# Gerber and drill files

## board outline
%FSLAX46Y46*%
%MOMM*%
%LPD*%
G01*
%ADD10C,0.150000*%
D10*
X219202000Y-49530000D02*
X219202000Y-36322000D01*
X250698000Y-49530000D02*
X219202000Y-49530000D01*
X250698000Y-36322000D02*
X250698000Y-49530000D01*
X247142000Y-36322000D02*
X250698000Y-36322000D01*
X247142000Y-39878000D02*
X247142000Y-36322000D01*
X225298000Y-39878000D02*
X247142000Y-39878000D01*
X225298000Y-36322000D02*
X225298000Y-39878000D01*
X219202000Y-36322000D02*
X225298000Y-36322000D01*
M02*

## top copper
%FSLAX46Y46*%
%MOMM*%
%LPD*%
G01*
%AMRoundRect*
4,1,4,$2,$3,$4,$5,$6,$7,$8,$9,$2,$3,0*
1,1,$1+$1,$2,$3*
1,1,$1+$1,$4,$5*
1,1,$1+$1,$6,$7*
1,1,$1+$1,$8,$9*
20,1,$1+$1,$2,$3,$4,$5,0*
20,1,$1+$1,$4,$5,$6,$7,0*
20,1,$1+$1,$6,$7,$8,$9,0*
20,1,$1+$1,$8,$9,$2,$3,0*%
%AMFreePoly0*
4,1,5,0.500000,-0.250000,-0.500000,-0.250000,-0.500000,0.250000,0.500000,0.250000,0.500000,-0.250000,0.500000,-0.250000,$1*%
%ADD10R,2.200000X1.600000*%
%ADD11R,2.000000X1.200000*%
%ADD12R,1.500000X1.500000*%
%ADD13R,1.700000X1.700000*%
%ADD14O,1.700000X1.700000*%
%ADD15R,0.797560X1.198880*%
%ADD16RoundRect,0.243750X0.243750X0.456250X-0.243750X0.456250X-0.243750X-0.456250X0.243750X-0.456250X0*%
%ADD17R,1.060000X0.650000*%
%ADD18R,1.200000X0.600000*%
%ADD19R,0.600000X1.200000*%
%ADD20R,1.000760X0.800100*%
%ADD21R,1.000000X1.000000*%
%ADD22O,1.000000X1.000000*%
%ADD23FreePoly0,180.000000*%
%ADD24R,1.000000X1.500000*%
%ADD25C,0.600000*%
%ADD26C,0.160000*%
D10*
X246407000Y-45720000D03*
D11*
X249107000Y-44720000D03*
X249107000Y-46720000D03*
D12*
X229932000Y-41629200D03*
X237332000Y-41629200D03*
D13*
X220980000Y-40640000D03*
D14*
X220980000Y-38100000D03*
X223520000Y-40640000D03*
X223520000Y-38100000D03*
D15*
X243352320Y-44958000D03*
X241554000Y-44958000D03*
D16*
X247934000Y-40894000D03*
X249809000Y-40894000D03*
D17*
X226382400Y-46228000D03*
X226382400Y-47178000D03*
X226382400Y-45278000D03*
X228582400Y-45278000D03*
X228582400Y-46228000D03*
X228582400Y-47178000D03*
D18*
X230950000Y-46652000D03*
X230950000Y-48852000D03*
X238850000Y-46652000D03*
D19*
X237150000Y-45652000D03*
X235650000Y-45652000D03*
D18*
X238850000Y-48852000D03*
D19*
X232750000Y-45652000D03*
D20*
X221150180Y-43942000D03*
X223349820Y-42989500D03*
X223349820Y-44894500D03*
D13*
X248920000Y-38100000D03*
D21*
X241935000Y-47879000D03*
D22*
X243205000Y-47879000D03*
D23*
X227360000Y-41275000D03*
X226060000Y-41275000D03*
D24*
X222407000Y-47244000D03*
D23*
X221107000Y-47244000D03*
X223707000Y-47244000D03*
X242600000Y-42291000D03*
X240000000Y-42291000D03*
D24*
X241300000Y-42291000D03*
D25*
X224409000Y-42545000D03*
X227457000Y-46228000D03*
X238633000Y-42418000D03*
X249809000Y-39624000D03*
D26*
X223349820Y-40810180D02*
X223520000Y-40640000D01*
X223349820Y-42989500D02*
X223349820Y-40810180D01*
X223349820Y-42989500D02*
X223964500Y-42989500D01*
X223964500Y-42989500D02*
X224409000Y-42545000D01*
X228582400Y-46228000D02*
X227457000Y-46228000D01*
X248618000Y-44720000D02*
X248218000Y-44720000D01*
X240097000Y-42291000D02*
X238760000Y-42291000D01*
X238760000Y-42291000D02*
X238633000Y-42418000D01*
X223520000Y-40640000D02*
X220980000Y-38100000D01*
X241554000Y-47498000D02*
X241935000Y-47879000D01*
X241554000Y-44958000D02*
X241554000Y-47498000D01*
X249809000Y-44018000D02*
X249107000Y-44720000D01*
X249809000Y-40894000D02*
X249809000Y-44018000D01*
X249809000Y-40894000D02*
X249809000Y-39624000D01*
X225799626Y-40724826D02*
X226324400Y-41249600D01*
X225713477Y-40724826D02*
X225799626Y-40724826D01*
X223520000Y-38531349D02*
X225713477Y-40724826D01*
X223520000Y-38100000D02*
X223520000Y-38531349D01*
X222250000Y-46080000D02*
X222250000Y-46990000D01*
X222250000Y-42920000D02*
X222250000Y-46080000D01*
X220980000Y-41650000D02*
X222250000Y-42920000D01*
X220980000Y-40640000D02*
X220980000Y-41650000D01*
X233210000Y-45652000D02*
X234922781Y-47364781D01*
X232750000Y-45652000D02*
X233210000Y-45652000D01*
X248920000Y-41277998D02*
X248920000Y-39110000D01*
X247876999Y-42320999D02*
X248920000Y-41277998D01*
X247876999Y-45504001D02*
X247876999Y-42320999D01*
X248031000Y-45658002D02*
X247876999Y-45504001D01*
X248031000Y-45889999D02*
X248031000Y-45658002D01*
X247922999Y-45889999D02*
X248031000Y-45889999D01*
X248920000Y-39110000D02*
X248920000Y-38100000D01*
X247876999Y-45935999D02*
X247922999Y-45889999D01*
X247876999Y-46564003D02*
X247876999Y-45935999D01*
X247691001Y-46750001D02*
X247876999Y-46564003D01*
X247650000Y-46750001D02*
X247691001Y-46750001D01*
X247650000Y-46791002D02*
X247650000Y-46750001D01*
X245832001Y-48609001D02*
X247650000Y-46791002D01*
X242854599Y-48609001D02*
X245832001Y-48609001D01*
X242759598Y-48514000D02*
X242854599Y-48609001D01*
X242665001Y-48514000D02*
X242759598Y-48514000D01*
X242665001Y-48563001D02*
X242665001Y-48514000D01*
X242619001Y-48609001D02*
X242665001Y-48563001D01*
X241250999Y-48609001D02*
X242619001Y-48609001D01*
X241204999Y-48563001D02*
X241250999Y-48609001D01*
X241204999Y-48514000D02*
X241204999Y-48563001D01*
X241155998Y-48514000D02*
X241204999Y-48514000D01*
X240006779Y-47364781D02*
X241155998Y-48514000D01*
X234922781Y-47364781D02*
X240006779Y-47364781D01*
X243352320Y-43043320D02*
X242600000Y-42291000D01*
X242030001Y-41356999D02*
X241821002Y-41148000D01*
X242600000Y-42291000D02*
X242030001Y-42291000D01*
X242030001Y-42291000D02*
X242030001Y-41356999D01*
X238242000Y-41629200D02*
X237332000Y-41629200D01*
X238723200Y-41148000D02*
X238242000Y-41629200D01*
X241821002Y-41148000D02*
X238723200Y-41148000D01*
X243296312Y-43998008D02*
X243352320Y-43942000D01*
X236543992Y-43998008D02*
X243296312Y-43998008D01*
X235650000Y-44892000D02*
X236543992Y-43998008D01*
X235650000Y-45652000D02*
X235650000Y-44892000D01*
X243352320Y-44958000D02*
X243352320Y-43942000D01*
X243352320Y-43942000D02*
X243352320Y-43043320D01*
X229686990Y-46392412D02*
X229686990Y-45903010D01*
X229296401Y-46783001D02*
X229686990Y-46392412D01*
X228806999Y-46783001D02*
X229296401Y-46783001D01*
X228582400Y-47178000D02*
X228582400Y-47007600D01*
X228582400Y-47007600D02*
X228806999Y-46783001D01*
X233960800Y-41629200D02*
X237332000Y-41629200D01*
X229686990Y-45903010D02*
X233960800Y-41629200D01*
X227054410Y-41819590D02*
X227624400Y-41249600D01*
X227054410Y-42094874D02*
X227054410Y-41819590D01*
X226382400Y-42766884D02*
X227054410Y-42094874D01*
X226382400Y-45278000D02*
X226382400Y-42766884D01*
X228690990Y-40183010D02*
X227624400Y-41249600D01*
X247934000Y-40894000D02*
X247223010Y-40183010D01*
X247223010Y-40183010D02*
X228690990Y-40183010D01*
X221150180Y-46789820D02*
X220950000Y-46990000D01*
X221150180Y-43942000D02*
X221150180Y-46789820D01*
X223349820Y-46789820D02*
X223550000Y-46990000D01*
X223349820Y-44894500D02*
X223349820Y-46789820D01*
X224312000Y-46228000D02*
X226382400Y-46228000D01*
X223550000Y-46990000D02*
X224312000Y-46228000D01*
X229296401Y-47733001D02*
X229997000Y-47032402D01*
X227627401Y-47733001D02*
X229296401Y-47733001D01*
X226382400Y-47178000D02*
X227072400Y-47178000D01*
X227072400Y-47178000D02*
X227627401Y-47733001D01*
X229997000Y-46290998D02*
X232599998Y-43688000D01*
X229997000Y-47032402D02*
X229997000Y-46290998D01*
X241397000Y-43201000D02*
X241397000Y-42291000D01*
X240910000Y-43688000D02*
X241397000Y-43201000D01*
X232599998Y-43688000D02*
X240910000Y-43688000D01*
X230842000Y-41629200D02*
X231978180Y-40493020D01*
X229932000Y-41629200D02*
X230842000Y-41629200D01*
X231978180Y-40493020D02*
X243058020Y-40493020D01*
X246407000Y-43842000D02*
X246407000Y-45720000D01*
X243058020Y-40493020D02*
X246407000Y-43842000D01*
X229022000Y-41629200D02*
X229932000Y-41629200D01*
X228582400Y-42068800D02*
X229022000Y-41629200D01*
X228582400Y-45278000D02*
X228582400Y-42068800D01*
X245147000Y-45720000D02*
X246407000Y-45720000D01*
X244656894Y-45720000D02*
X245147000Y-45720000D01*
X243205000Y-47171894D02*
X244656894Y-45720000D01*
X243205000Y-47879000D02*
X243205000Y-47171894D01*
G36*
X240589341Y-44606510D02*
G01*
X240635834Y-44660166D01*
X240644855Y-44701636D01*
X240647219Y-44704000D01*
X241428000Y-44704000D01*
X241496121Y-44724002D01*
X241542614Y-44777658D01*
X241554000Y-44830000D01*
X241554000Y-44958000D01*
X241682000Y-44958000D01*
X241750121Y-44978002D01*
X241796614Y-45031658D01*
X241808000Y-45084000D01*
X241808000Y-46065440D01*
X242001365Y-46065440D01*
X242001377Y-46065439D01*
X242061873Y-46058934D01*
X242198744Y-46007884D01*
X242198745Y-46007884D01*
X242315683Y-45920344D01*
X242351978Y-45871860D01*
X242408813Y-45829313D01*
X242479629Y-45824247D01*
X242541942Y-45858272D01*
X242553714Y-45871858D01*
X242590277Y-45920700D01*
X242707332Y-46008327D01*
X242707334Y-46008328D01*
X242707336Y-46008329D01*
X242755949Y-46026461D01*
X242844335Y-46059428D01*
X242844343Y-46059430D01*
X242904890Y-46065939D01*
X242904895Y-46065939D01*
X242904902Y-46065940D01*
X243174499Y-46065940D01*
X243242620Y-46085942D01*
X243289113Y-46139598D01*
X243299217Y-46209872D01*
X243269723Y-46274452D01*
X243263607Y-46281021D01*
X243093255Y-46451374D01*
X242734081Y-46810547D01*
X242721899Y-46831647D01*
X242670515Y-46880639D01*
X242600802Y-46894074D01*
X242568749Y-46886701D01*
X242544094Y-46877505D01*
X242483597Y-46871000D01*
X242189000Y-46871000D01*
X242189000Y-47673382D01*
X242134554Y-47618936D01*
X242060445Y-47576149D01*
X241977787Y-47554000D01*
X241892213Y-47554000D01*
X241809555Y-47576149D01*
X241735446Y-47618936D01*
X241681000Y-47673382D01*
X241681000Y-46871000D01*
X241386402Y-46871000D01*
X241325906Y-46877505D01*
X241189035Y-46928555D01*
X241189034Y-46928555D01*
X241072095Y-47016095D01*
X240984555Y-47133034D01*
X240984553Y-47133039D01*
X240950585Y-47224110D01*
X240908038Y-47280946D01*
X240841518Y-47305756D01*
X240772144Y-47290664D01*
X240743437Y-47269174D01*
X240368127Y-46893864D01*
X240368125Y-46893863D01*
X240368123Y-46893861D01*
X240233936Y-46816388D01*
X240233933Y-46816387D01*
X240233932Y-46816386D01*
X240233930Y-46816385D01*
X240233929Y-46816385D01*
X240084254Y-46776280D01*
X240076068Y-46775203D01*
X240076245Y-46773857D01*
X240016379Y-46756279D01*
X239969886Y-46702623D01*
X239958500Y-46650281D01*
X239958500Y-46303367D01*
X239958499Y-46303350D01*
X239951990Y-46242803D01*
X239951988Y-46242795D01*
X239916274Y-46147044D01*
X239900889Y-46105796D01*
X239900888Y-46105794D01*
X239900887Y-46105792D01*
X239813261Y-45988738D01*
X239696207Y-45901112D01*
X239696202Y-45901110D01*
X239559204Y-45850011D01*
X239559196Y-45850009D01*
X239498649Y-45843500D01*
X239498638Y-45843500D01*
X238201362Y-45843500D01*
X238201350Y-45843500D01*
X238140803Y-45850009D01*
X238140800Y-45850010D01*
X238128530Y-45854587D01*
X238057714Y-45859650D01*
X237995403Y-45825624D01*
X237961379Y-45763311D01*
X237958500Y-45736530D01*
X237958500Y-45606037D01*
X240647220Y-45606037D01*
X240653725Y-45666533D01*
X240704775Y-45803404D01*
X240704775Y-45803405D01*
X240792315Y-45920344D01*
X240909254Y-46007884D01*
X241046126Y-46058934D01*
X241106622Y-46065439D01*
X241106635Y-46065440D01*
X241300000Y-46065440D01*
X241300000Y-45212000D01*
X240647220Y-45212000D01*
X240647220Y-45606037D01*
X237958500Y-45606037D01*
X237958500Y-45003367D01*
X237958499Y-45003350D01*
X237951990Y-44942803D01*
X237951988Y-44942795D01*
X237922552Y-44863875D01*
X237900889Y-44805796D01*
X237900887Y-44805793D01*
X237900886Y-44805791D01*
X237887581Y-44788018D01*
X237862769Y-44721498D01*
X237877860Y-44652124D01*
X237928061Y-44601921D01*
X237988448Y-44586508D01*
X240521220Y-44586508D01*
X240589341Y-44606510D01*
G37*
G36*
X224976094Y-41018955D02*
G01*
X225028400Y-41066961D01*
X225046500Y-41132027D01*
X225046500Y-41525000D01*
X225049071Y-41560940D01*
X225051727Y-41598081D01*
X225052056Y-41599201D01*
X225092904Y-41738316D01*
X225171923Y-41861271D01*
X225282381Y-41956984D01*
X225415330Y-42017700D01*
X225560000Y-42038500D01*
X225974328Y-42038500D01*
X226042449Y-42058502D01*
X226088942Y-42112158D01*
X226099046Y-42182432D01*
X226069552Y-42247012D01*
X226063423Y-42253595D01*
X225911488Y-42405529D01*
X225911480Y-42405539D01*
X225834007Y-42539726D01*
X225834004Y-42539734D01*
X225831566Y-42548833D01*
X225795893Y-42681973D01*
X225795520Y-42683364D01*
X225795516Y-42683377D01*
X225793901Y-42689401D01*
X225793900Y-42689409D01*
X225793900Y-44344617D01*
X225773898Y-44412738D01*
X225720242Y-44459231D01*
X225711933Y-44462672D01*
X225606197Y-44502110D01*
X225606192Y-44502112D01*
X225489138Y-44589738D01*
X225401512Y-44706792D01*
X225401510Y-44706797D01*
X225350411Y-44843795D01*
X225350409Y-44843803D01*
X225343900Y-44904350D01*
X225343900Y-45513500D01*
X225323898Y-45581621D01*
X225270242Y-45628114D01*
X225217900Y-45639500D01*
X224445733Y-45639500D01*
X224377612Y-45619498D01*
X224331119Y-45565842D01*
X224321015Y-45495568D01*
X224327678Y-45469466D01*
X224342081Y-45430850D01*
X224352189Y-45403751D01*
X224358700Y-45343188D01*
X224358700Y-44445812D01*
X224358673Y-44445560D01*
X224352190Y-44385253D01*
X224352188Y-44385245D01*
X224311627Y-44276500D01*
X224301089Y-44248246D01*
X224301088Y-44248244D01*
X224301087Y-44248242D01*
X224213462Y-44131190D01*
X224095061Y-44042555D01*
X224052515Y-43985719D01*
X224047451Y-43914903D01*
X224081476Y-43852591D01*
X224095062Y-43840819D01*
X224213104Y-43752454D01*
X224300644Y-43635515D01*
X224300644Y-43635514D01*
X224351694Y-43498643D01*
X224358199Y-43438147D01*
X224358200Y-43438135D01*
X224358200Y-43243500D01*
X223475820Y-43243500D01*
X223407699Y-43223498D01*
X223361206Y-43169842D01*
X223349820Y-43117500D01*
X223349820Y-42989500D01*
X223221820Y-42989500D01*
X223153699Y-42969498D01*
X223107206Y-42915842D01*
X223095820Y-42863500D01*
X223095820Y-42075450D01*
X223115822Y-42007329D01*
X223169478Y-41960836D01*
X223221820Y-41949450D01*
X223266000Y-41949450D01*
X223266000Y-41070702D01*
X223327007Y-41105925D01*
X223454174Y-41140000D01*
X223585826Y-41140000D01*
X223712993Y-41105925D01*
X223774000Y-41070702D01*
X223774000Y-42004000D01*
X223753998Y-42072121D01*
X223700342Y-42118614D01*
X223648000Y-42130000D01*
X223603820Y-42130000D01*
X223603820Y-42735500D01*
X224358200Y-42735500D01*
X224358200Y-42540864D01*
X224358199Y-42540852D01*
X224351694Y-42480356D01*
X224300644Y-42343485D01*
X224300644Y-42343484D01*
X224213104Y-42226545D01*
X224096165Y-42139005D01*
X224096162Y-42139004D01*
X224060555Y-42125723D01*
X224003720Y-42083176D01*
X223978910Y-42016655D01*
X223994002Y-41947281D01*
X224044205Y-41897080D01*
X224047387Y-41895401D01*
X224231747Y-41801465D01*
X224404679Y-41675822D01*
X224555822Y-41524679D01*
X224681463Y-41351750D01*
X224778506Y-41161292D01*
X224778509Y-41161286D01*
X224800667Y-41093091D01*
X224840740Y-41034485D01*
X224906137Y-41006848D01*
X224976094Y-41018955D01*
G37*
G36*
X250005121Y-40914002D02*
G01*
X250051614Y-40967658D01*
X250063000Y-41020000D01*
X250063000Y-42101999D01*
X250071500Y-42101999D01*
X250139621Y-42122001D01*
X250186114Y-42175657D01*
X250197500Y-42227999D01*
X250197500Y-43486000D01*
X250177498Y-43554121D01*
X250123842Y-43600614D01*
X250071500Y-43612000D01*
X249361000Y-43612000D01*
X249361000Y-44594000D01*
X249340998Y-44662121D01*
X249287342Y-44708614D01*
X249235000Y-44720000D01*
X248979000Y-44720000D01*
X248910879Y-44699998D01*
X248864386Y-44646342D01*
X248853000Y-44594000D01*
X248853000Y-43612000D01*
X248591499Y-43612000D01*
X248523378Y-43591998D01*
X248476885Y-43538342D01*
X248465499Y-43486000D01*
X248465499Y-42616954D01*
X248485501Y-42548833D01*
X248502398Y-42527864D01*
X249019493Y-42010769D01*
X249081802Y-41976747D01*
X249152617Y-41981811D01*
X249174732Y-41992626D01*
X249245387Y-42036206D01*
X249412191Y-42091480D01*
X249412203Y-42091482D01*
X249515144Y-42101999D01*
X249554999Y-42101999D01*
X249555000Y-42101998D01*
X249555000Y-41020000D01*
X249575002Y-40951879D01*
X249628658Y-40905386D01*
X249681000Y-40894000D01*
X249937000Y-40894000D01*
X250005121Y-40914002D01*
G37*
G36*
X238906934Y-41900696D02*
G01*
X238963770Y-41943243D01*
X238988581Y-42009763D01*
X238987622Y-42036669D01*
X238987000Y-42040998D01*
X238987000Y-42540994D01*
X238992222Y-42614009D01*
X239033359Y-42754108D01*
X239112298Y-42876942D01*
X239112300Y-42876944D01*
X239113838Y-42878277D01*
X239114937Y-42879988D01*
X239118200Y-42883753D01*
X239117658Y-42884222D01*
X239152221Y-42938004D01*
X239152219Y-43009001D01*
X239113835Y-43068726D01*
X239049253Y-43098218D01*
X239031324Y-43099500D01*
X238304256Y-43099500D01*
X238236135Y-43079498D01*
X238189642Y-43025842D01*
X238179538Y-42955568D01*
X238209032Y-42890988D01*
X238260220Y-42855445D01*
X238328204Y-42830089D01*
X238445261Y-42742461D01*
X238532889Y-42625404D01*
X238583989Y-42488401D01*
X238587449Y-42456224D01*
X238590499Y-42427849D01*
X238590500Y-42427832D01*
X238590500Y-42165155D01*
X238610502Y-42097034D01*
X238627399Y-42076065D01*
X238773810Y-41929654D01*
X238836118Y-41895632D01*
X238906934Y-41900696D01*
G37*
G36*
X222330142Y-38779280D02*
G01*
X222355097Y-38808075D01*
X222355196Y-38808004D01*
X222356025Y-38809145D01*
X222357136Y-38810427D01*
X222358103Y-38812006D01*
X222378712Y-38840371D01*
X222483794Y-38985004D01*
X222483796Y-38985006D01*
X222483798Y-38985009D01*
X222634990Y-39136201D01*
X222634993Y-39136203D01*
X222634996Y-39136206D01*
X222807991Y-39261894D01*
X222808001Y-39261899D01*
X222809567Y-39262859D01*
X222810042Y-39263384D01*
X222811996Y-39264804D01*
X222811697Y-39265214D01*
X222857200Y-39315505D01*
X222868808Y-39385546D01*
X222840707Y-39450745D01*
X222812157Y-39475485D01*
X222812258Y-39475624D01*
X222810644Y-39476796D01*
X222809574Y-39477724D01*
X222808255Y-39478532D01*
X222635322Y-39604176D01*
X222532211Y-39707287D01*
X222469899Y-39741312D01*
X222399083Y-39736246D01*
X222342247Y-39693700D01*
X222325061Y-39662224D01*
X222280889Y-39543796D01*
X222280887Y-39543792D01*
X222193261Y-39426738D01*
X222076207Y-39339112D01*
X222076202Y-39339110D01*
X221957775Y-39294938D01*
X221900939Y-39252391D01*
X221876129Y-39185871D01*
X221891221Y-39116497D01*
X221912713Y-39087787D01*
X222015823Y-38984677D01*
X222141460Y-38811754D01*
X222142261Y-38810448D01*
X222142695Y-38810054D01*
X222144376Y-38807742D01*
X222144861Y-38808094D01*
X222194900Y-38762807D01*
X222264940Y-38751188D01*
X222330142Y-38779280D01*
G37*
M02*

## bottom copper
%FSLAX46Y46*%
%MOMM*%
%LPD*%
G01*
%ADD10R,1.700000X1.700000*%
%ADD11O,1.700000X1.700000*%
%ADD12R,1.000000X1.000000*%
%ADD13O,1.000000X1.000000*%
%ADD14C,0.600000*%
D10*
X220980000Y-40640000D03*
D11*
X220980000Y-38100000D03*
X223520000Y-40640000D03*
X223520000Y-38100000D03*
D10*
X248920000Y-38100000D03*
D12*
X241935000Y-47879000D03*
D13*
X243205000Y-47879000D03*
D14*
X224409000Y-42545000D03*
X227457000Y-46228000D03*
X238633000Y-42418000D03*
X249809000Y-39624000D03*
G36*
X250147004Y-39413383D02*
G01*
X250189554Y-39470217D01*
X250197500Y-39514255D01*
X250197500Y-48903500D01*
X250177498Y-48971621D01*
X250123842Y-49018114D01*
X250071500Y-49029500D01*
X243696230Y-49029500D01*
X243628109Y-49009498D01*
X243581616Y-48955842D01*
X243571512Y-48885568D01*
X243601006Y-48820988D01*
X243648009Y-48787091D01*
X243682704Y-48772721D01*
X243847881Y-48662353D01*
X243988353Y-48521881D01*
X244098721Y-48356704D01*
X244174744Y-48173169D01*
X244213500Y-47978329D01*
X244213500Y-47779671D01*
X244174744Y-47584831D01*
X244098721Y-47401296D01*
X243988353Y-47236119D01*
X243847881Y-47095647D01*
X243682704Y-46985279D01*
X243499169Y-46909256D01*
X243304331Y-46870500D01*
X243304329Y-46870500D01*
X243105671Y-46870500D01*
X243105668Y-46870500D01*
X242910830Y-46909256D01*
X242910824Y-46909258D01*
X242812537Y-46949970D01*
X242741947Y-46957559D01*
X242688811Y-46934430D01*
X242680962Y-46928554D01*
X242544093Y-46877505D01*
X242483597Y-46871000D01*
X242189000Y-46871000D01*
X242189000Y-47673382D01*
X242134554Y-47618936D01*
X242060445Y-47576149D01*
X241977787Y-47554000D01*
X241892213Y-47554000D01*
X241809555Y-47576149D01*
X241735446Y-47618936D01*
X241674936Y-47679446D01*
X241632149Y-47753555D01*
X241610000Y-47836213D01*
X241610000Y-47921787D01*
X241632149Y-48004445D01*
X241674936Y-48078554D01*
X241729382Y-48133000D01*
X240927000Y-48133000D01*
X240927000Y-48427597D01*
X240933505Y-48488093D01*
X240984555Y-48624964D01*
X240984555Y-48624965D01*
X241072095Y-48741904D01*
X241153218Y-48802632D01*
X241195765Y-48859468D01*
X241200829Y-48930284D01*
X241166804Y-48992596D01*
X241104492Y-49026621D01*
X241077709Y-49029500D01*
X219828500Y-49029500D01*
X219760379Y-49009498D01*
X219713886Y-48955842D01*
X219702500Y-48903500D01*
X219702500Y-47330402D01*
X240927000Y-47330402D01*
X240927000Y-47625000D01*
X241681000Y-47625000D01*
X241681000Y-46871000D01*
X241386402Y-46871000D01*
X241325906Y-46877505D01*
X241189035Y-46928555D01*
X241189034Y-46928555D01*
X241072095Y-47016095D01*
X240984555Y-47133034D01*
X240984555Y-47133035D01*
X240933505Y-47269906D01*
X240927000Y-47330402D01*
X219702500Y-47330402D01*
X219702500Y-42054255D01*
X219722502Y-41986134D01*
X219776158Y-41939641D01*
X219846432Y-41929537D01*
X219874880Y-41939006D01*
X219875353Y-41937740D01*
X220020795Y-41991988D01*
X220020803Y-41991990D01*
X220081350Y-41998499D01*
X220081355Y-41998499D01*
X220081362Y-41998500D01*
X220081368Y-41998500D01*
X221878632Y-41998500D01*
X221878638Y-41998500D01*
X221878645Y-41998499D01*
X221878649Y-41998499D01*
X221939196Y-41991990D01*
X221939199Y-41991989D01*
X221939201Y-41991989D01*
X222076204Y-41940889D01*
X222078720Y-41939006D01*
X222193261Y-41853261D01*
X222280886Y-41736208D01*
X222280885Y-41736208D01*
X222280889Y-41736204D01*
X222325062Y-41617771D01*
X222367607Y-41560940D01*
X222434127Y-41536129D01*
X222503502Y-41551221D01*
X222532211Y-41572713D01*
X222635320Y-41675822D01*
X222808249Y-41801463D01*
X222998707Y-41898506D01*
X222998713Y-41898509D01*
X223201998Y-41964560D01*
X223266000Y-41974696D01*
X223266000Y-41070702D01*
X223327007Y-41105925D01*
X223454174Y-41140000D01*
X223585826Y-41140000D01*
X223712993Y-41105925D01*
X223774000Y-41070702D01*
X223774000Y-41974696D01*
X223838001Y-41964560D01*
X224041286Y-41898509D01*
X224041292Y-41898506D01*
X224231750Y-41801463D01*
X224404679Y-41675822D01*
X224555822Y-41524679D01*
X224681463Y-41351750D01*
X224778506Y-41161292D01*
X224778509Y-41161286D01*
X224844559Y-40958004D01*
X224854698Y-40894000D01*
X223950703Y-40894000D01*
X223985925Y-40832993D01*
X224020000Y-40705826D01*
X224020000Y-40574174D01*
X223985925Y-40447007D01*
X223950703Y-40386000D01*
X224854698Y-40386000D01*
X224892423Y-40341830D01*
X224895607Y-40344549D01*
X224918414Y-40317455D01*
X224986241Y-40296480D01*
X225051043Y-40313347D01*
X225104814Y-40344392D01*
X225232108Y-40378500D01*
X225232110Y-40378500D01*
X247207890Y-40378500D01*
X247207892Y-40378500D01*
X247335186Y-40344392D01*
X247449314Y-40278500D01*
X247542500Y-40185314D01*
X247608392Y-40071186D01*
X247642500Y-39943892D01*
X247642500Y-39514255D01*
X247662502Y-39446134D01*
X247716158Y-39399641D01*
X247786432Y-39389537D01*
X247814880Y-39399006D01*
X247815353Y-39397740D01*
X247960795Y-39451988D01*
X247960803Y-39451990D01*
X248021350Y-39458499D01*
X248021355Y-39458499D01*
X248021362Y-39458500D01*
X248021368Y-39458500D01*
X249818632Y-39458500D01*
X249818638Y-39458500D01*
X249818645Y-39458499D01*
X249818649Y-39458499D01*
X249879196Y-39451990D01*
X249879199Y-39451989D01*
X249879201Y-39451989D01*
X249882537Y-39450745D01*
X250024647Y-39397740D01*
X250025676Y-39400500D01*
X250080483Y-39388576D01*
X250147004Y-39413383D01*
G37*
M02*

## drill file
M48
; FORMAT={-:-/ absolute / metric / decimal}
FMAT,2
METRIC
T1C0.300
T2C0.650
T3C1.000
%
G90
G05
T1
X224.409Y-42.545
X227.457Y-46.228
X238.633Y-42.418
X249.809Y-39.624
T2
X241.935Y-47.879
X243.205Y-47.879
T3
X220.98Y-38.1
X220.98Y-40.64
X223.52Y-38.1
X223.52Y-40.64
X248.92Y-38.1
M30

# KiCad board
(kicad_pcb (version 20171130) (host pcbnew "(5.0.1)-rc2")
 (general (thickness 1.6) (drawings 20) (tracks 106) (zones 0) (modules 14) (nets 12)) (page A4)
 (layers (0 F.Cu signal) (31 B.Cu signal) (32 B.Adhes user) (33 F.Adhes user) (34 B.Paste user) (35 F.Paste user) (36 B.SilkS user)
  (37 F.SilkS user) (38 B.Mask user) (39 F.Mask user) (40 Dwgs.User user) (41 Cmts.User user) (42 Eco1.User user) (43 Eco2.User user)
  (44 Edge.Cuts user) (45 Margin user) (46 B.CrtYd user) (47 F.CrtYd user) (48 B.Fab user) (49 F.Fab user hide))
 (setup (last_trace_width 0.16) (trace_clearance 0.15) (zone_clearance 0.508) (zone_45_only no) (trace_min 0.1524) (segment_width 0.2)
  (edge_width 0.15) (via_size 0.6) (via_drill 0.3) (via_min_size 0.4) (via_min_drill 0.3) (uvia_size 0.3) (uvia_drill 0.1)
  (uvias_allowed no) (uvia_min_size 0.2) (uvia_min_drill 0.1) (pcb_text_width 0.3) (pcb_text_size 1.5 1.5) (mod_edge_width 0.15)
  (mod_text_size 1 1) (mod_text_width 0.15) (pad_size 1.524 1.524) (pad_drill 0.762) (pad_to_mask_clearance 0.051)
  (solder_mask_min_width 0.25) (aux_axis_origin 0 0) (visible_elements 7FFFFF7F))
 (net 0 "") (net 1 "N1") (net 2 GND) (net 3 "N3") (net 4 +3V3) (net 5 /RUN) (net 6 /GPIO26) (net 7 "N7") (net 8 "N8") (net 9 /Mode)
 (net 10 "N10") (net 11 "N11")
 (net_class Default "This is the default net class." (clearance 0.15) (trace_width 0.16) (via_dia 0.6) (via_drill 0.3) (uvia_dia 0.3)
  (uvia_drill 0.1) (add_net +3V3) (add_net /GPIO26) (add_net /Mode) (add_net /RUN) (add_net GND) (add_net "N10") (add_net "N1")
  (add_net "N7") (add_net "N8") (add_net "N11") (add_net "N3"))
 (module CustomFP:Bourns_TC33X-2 (layer F.Cu) (at 246.507 45.72 90)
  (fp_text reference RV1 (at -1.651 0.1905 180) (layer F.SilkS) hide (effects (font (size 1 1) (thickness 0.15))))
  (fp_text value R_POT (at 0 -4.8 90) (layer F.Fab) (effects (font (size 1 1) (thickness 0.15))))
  (pad 1 smd rect (at 0 -0.1 90) (size 1.6 2.2) (layers F.Cu F.Paste F.Mask) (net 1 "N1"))
  (pad 2 smd rect (at 1 2.6 90) (size 1.2 2) (layers F.Cu F.Paste F.Mask) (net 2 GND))
  (pad 3 smd rect (at -1 2.6 90) (size 1.2 2) (layers F.Cu F.Paste F.Mask) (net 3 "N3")))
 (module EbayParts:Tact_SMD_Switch (layer F.Cu) (at 230.632 43.1292)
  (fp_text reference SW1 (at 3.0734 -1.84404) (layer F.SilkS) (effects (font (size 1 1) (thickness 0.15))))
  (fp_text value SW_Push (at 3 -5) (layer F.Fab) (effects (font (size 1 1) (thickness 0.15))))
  (pad 1 smd rect (at -0.7 -1.5) (size 1.5 1.5) (layers F.Cu F.Paste F.Mask) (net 1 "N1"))
  (pad 2 smd rect (at 6.7 -1.5) (size 1.5 1.5) (layers F.Cu F.Paste F.Mask) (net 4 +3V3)))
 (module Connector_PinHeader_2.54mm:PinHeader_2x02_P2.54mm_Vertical (layer F.Cu) (at 220.98 40.64 90)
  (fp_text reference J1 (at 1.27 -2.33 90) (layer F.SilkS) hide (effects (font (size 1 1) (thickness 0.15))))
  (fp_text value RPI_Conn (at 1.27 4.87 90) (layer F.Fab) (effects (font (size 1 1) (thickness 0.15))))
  (pad 1 thru_hole rect (at 0 0 90) (size 1.7 1.7) (drill 1) (layers *.Cu *.Mask) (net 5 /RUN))
  (pad 2 thru_hole oval (at 2.54 0 90) (size 1.7 1.7) (drill 1) (layers *.Cu *.Mask) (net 2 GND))
  (pad 3 thru_hole oval (at 0 2.54 90) (size 1.7 1.7) (drill 1) (layers *.Cu *.Mask) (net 2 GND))
  (pad 4 thru_hole oval (at 2.54 2.54 90) (size 1.7 1.7) (drill 1) (layers *.Cu *.Mask) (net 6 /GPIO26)))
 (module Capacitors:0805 (layer F.Cu) (at 242.45316 44.958)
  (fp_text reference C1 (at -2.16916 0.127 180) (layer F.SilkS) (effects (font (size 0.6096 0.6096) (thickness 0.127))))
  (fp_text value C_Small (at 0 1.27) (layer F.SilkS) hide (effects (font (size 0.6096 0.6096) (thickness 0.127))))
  (pad 2 smd rect (at 0.89916 0) (size 0.79756 1.19888) (layers F.Cu F.Paste F.Mask) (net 4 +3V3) (solder_mask_margin 0.1016))
  (pad 1 smd rect (at -0.89916 0) (size 0.79756 1.19888) (layers F.Cu F.Paste F.Mask) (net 2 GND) (solder_mask_margin 0.1016)))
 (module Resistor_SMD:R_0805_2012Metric (layer F.Cu) (at 248.8715 40.894 180)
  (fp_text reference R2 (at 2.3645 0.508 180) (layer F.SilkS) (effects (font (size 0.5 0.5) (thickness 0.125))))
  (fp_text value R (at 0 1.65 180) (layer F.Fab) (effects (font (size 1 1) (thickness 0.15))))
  (pad 2 smd roundrect (at 0.9375 0 180) (size 0.975 1.4) (layers F.Cu F.Paste F.Mask) (roundrect_rratio 0.25) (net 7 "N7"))
  (pad 1 smd roundrect (at -0.9375 0 180) (size 0.975 1.4) (layers F.Cu F.Paste F.Mask) (roundrect_rratio 0.25) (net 2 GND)))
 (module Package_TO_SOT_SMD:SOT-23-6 (layer F.Cu) (at 227.4824 46.228 180)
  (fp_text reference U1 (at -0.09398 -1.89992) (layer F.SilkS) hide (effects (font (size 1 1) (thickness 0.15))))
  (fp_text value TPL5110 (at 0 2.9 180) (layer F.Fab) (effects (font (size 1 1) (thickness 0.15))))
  (pad 5 smd rect (at 1.1 0 180) (size 1.06 0.65) (layers F.Cu F.Paste F.Mask) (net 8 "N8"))
  (pad 6 smd rect (at 1.1 -0.95 180) (size 1.06 0.65) (layers F.Cu F.Paste F.Mask) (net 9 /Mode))
  (pad 4 smd rect (at 1.1 0.95 180) (size 1.06 0.65) (layers F.Cu F.Paste F.Mask) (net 7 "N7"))
  (pad 3 smd rect (at -1.1 0.95 180) (size 1.06 0.65) (layers F.Cu F.Paste F.Mask) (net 1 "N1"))
  (pad 2 smd rect (at -1.1 0 180) (size 1.06 0.65) (layers F.Cu F.Paste F.Mask) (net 2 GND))
  (pad 1 smd rect (at -1.1 -0.95 180) (size 1.06 0.65) (layers F.Cu F.Paste F.Mask) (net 4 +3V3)))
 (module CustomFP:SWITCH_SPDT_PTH (layer F.Cu) (at 234.95 47.752 90)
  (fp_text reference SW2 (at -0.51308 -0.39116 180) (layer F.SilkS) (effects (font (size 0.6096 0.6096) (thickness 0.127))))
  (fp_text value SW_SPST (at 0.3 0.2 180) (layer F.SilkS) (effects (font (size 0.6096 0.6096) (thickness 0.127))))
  (pad "" smd rect (at 1.1 -4 180) (size 1.2 0.6) (layers F.Cu F.Paste F.Mask) (solder_mask_margin 0.1016))
  (pad "" smd rect (at -1.1 -4 180) (size 1.2 0.6) (layers F.Cu F.Paste F.Mask) (solder_mask_margin 0.1016))
  (pad "" smd rect (at 1.1 3.9 180) (size 1.2 0.6) (layers F.Cu F.Paste F.Mask) (solder_mask_margin 0.1016))
  (pad 3 smd rect (at 2.1 2.2 90) (size 1.2 0.6) (layers F.Cu F.Paste F.Mask) (solder_mask_margin 0.1016))
  (pad 2 smd rect (at 2.1 0.7 90) (size 1.2 0.6) (layers F.Cu F.Paste F.Mask) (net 4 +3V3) (solder_mask_margin 0.1016))
  (pad "" smd rect (at -1.1 3.9 180) (size 1.2 0.6) (layers F.Cu F.Paste F.Mask) (solder_mask_margin 0.1016))
  (pad 1 smd rect (at 2.1 -2.2 90) (size 1.2 0.6) (layers F.Cu F.Paste F.Mask) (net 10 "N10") (solder_mask_margin 0.1016)))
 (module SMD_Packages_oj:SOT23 (layer F.Cu) (at 222.25 43.942 90)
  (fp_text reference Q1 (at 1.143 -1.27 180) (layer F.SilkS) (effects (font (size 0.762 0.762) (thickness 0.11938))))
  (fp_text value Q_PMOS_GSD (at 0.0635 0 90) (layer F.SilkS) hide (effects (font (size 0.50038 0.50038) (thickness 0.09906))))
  (pad 3 smd rect (at 0 -1.09982 90) (size 0.8001 1.00076) (layers F.Cu F.Paste F.Mask) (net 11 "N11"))
  (pad 2 smd rect (at 0.9525 1.09982 90) (size 0.8001 1.00076) (layers F.Cu F.Paste F.Mask) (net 2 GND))
  (pad 1 smd rect (at -0.9525 1.09982 90) (size 0.8001 1.00076) (layers F.Cu F.Paste F.Mask) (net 8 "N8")))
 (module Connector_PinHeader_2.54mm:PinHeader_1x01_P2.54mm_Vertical (layer F.Cu) (at 248.92 38.1)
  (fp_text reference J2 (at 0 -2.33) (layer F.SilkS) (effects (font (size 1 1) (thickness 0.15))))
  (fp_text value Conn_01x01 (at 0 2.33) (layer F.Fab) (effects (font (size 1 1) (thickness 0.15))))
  (pad 1 thru_hole rect (at 0 0) (size 1.7 1.7) (drill 1) (layers *.Cu *.Mask) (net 10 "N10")))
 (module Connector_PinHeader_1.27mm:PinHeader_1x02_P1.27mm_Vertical (layer F.Cu) (at 241.935 47.879 90)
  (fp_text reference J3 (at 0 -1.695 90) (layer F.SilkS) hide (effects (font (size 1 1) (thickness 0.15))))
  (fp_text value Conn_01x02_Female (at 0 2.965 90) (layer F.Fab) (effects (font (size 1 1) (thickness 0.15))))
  (pad 1 thru_hole rect (at 0 0 90) (size 1 1) (drill 0.65) (layers *.Cu *.Mask) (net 2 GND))
  (pad 2 thru_hole oval (at 0 1.27 90) (size 1 1) (drill 0.65) (layers *.Cu *.Mask) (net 1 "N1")))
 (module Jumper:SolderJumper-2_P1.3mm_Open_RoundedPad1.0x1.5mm (layer F.Cu) (at 226.71 41.275 180)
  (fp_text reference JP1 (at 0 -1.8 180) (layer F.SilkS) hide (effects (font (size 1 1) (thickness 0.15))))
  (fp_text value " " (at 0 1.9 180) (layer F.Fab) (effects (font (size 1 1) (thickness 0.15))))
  (pad 1 smd custom (at -0.65 0 180) (size 1 0.5) (layers F.Cu F.Mask) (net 7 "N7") (zone_connect 0)
   (options (clearance outline) (anchor rect)) (primitives))
  (pad 2 smd custom (at 0.65 0 180) (size 1 0.5) (layers F.Cu F.Mask) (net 6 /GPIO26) (zone_connect 0)
   (options (clearance outline) (anchor rect)) (primitives)))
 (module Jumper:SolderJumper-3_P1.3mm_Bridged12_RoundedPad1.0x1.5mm (layer F.Cu) (at 222.407 47.244 180)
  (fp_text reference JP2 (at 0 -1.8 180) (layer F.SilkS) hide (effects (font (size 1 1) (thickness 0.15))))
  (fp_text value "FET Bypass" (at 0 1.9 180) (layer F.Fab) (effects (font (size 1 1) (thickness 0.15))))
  (pad 2 smd rect (at 0 0 180) (size 1 1.5) (layers F.Cu F.Mask) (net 5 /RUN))
  (pad 3 smd custom (at 1.3 0 180) (size 1 0.5) (layers F.Cu F.Mask) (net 11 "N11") (zone_connect 0)
   (options (clearance outline) (anchor rect)) (primitives))
  (pad 1 smd custom (at -1.3 0 180) (size 1 0.5) (layers F.Cu F.Mask) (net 8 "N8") (zone_connect 0)
   (options (clearance outline) (anchor rect)) (primitives)))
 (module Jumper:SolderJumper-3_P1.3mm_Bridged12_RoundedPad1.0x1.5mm (layer F.Cu) (at 241.3 42.291 180)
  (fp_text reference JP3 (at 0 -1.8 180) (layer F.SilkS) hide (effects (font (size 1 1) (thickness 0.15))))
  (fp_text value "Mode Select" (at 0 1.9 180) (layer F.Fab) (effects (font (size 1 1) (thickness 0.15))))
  (pad 1 smd custom (at -1.3 0 180) (size 1 0.5) (layers F.Cu F.Mask) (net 4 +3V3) (zone_connect 0)
   (options (clearance outline) (anchor rect)) (primitives))
  (pad 3 smd custom (at 1.3 0 180) (size 1 0.5) (layers F.Cu F.Mask) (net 2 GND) (zone_connect 0)
   (options (clearance outline) (anchor rect)) (primitives))
  (pad 2 smd rect (at 0 0 180) (size 1 1.5) (layers F.Cu F.Mask) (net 9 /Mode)))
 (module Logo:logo (layer B.Cu) (at 226.949 45.339 180)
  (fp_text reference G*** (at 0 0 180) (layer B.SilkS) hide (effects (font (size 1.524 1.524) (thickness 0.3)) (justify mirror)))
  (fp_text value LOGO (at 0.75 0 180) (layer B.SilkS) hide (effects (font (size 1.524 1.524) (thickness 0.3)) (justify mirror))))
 (gr_line (start 219.202 49.53) (end 219.202 36.322) (layer Edge.Cuts) (width 0.15))
 (gr_line (start 250.698 49.53) (end 219.202 49.53) (layer Edge.Cuts) (width 0.15))
 (gr_line (start 250.698 36.322) (end 250.698 49.53) (layer Edge.Cuts) (width 0.15))
 (gr_line (start 247.142 36.322) (end 250.698 36.322) (layer Edge.Cuts) (width 0.15))
 (gr_line (start 247.142 39.878) (end 247.142 36.322) (layer Edge.Cuts) (width 0.15))
 (gr_line (start 225.298 39.878) (end 247.142 39.878) (layer Edge.Cuts) (width 0.15))
 (gr_line (start 225.298 36.322) (end 225.298 39.878) (layer Edge.Cuts) (width 0.15))
 (gr_line (start 219.202 36.322) (end 225.298 36.322) (layer Edge.Cuts) (width 0.15))
 (segment (start 223.34982 40.81018) (end 223.52 40.64) (width 0.16) (layer F.Cu) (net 2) (status 30))
 (segment (start 223.34982 42.9895) (end 223.34982 40.81018) (width 0.16) (layer F.Cu) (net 2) (status 30))
 (via (at 224.409 42.545) (size 0.6) (drill 0.3) (layers F.Cu B.Cu) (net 2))
 (segment (start 223.34982 42.9895) (end 223.9645 42.9895) (width 0.16) (layer F.Cu) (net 2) (status 10))
 (segment (start 223.9645 42.9895) (end 224.409 42.545) (width 0.16) (layer F.Cu) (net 2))
 (via (at 227.457 46.228) (size 0.6) (drill 0.3) (layers F.Cu B.Cu) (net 2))
 (segment (start 228.5824 46.228) (end 227.457 46.228) (width 0.16) (layer F.Cu) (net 2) (status 10))
 (segment (start 248.618 44.72) (end 248.218 44.72) (width 0.16) (layer F.Cu) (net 2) (status 30))
 (via (at 238.633 42.418) (size 0.6) (drill 0.3) (layers F.Cu B.Cu) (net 2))
 (segment (start 240.097 42.291) (end 238.76 42.291) (width 0.16) (layer F.Cu) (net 2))
 (segment (start 238.76 42.291) (end 238.633 42.418) (width 0.16) (layer F.Cu) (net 2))
 (segment (start 223.52 40.64) (end 220.98 38.1) (width 0.16) (layer F.Cu) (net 2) (status 30))
 (segment (start 241.554 47.498) (end 241.935 47.879) (width 0.16) (layer F.Cu) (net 2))
 (segment (start 241.554 44.958) (end 241.554 47.498) (width 0.16) (layer F.Cu) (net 2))
 (segment (start 249.809 44.018) (end 249.107 44.72) (width 0.16) (layer F.Cu) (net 2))
 (segment (start 249.809 40.894) (end 249.809 44.018) (width 0.16) (layer F.Cu) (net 2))
 (via (at 249.809 39.624) (size 0.6) (drill 0.3) (layers F.Cu B.Cu) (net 2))
 (segment (start 249.809 40.894) (end 249.809 39.624) (width 0.16) (layer F.Cu) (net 2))
 (segment (start 225.799626 40.724826) (end 226.3244 41.2496) (width 0.16) (layer F.Cu) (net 6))
 (segment (start 225.713477 40.724826) (end 225.799626 40.724826) (width 0.16) (layer F.Cu) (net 6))
 (segment (start 223.52 38.531349) (end 225.713477 40.724826) (width 0.16) (layer F.Cu) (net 6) (status 10))
 (segment (start 223.52 38.1) (end 223.52 38.531349) (width 0.16) (layer F.Cu) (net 6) (status 30))
 (segment (start 222.25 46.08) (end 222.25 46.99) (width 0.16) (layer F.Cu) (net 5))
 (segment (start 222.25 42.92) (end 222.25 46.08) (width 0.16) (layer F.Cu) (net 5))
 (segment (start 220.98 41.65) (end 222.25 42.92) (width 0.16) (layer F.Cu) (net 5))
 (segment (start 220.98 40.64) (end 220.98 41.65) (width 0.16) (layer F.Cu) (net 5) (status 10))
 (segment (start 233.21 45.652) (end 234.922781 47.364781) (width 0.16) (layer F.Cu) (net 10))
 (segment (start 232.75 45.652) (end 233.21 45.652) (width 0.16) (layer F.Cu) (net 10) (status 10))
 (segment (start 248.92 41.277998) (end 248.92 39.11) (width 0.16) (layer F.Cu) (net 10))
 (segment (start 247.876999 42.320999) (end 248.92 41.277998) (width 0.16) (layer F.Cu) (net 10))
 (segment (start 247.876999 45.504001) (end 247.876999 42.320999) (width 0.16) (layer F.Cu) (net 10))
 (segment (start 248.031 45.658002) (end 247.876999 45.504001) (width 0.16) (layer F.Cu) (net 10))
 (segment (start 248.031 45.889999) (end 248.031 45.658002) (width 0.16) (layer F.Cu) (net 10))
 (segment (start 247.922999 45.889999) (end 248.031 45.889999) (width 0.16) (layer F.Cu) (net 10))
 (segment (start 248.92 39.11) (end 248.92 38.1) (width 0.16) (layer F.Cu) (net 10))
 (segment (start 247.876999 45.935999) (end 247.922999 45.889999) (width 0.16) (layer F.Cu) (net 10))
 (segment (start 247.876999 46.564003) (end 247.876999 45.935999) (width 0.16) (layer F.Cu) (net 10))
 (segment (start 247.691001 46.750001) (end 247.876999 46.564003) (width 0.16) (layer F.Cu) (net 10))
 (segment (start 247.65 46.750001) (end 247.691001 46.750001) (width 0.16) (layer F.Cu) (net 10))
 (segment (start 247.65 46.791002) (end 247.65 46.750001) (width 0.16) (layer F.Cu) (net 10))
 (segment (start 245.832001 48.609001) (end 247.65 46.791002) (width 0.16) (layer F.Cu) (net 10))
 (segment (start 242.854599 48.609001) (end 245.832001 48.609001) (width 0.16) (layer F.Cu) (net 10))
 (segment (start 242.759598 48.514) (end 242.854599 48.609001) (width 0.16) (layer F.Cu) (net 10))
 (segment (start 242.665001 48.514) (end 242.759598 48.514) (width 0.16) (layer F.Cu) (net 10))
 (segment (start 242.665001 48.563001) (end 242.665001 48.514) (width 0.16) (layer F.Cu) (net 10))
 (segment (start 242.619001 48.609001) (end 242.665001 48.563001) (width 0.16) (layer F.Cu) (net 10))
 (segment (start 241.250999 48.609001) (end 242.619001 48.609001) (width 0.16) (layer F.Cu) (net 10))
 (segment (start 241.204999 48.563001) (end 241.250999 48.609001) (width 0.16) (layer F.Cu) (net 10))
 (segment (start 241.204999 48.514) (end 241.204999 48.563001) (width 0.16) (layer F.Cu) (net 10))
 (segment (start 241.155998 48.514) (end 241.204999 48.514) (width 0.16) (layer F.Cu) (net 10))
 (segment (start 240.006779 47.364781) (end 241.155998 48.514) (width 0.16) (layer F.Cu) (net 10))
 (segment (start 234.922781 47.364781) (end 240.006779 47.364781) (width 0.16) (layer F.Cu) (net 10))
 (segment (start 243.35232 43.04332) (end 242.6 42.291) (width 0.16) (layer F.Cu) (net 4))
 (segment (start 242.030001 41.356999) (end 241.821002 41.148) (width 0.16) (layer F.Cu) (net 4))
 (segment (start 242.6 42.291) (end 242.030001 42.291) (width 0.16) (layer F.Cu) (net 4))
 (segment (start 242.030001 42.291) (end 242.030001 41.356999) (width 0.16) (layer F.Cu) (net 4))
 (segment (start 238.242 41.6292) (end 237.332 41.6292) (width 0.16) (layer F.Cu) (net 4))
 (segment (start 238.7232 41.148) (end 238.242 41.6292) (width 0.16) (layer F.Cu) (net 4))
 (segment (start 241.821002 41.148) (end 238.7232 41.148) (width 0.16) (layer F.Cu) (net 4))
 (segment (start 243.296312 43.998008) (end 243.35232 43.942) (width 0.16) (layer F.Cu) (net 4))
 (segment (start 236.543992 43.998008) (end 243.296312 43.998008) (width 0.16) (layer F.Cu) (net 4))
 (segment (start 235.65 44.892) (end 236.543992 43.998008) (width 0.16) (layer F.Cu) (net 4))
 (segment (start 235.65 45.652) (end 235.65 44.892) (width 0.16) (layer F.Cu) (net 4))
 (segment (start 243.35232 44.958) (end 243.35232 43.942) (width 0.16) (layer F.Cu) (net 4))
 (segment (start 243.35232 43.942) (end 243.35232 43.04332) (width 0.16) (layer F.Cu) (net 4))
 (segment (start 229.68699 46.392412) (end 229.68699 45.90301) (width 0.16) (layer F.Cu) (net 4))
 (segment (start 229.296401 46.783001) (end 229.68699 46.392412) (width 0.16) (layer F.Cu) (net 4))
 (segment (start 228.806999 46.783001) (end 229.296401 46.783001) (width 0.16) (layer F.Cu) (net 4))
 (segment (start 228.5824 47.178) (end 228.5824 47.0076) (width 0.16) (layer F.Cu) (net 4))
 (segment (start 228.5824 47.0076) (end 228.806999 46.783001) (width 0.16) (layer F.Cu) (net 4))
 (segment (start 233.9608 41.6292) (end 237.332 41.6292) (width 0.16) (layer F.Cu) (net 4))
 (segment (start 229.68699 45.90301) (end 233.9608 41.6292) (width 0.16) (layer F.Cu) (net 4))
 (segment (start 227.05441 41.81959) (end 227.6244 41.2496) (width 0.16) (layer F.Cu) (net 7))
 (segment (start 227.05441 42.094874) (end 227.05441 41.81959) (width 0.16) (layer F.Cu) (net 7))
 (segment (start 226.3824 42.766884) (end 227.05441 42.094874) (width 0.16) (layer F.Cu) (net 7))
 (segment (start 226.3824 45.278) (end 226.3824 42.766884) (width 0.16) (layer F.Cu) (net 7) (status 10))
 (segment (start 228.69099 40.18301) (end 227.6244 41.2496) (width 0.16) (layer F.Cu) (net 7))
 (segment (start 247.934 40.894) (end 247.22301 40.18301) (width 0.16) (layer F.Cu) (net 7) (status 10))
 (segment (start 247.22301 40.18301) (end 228.69099 40.18301) (width 0.16) (layer F.Cu) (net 7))
 (segment (start 221.15018 46.78982) (end 220.95 46.99) (width 0.16) (layer F.Cu) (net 11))
 (segment (start 221.15018 43.942) (end 221.15018 46.78982) (width 0.16) (layer F.Cu) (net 11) (status 10))
 (segment (start 223.34982 46.78982) (end 223.55 46.99) (width 0.16) (layer F.Cu) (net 8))
 (segment (start 223.34982 44.8945) (end 223.34982 46.78982) (width 0.16) (layer F.Cu) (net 8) (status 10))
 (segment (start 224.312 46.228) (end 226.3824 46.228) (width 0.16) (layer F.Cu) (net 8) (status 20))
 (segment (start 223.55 46.99) (end 224.312 46.228) (width 0.16) (layer F.Cu) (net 8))
 (segment (start 229.296401 47.733001) (end 229.997 47.032402) (width 0.16) (layer F.Cu) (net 9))
 (segment (start 227.627401 47.733001) (end 229.296401 47.733001) (width 0.16) (layer F.Cu) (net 9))
 (segment (start 226.3824 47.178) (end 227.0724 47.178) (width 0.16) (layer F.Cu) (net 9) (status 10))
 (segment (start 227.0724 47.178) (end 227.627401 47.733001) (width 0.16) (layer F.Cu) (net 9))
 (segment (start 229.997 46.290998) (end 232.599998 43.688) (width 0.16) (layer F.Cu) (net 9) (status 20))
 (segment (start 229.997 47.032402) (end 229.997 46.290998) (width 0.16) (layer F.Cu) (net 9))
 (segment (start 241.397 43.201) (end 241.397 42.291) (width 0.16) (layer F.Cu) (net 9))
 (segment (start 240.91 43.688) (end 241.397 43.201) (width 0.16) (layer F.Cu) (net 9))
 (segment (start 232.599998 43.688) (end 240.91 43.688) (width 0.16) (layer F.Cu) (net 9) (status 10))
 (segment (start 230.842 41.6292) (end 231.97818 40.49302) (width 0.16) (layer F.Cu) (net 1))
 (segment (start 229.932 41.6292) (end 230.842 41.6292) (width 0.16) (layer F.Cu) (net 1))
 (segment (start 231.97818 40.49302) (end 243.05802 40.49302) (width 0.16) (layer F.Cu) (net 1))
 (segment (start 246.407 43.842) (end 246.407 45.72) (width 0.16) (layer F.Cu) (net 1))
 (segment (start 243.05802 40.49302) (end 246.407 43.842) (width 0.16) (layer F.Cu) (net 1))
 (segment (start 229.022 41.6292) (end 229.932 41.6292) (width 0.16) (layer F.Cu) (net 1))
 (segment (start 228.5824 42.0688) (end 229.022 41.6292) (width 0.16) (layer F.Cu) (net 1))
 (segment (start 228.5824 45.278) (end 228.5824 42.0688) (width 0.16) (layer F.Cu) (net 1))
 (segment (start 245.147 45.72) (end 246.407 45.72) (width 0.16) (layer F.Cu) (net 1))
 (segment (start 244.656894 45.72) (end 245.147 45.72) (width 0.16) (layer F.Cu) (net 1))
 (segment (start 243.205 47.171894) (end 244.656894 45.72) (width 0.16) (layer F.Cu) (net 1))
 (segment (start 243.205 47.879) (end 243.205 47.171894) (width 0.16) (layer F.Cu) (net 1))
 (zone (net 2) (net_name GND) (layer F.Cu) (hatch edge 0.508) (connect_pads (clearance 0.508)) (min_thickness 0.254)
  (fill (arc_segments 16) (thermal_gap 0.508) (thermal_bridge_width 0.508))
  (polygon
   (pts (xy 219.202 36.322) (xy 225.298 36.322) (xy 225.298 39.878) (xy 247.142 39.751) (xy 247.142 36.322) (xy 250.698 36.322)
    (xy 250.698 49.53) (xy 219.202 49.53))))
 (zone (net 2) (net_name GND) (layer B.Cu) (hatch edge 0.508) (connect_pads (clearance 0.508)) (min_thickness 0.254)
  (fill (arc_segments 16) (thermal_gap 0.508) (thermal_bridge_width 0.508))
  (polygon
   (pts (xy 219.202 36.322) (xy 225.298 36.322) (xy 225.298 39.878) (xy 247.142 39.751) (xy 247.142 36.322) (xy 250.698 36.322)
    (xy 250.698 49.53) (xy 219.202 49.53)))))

